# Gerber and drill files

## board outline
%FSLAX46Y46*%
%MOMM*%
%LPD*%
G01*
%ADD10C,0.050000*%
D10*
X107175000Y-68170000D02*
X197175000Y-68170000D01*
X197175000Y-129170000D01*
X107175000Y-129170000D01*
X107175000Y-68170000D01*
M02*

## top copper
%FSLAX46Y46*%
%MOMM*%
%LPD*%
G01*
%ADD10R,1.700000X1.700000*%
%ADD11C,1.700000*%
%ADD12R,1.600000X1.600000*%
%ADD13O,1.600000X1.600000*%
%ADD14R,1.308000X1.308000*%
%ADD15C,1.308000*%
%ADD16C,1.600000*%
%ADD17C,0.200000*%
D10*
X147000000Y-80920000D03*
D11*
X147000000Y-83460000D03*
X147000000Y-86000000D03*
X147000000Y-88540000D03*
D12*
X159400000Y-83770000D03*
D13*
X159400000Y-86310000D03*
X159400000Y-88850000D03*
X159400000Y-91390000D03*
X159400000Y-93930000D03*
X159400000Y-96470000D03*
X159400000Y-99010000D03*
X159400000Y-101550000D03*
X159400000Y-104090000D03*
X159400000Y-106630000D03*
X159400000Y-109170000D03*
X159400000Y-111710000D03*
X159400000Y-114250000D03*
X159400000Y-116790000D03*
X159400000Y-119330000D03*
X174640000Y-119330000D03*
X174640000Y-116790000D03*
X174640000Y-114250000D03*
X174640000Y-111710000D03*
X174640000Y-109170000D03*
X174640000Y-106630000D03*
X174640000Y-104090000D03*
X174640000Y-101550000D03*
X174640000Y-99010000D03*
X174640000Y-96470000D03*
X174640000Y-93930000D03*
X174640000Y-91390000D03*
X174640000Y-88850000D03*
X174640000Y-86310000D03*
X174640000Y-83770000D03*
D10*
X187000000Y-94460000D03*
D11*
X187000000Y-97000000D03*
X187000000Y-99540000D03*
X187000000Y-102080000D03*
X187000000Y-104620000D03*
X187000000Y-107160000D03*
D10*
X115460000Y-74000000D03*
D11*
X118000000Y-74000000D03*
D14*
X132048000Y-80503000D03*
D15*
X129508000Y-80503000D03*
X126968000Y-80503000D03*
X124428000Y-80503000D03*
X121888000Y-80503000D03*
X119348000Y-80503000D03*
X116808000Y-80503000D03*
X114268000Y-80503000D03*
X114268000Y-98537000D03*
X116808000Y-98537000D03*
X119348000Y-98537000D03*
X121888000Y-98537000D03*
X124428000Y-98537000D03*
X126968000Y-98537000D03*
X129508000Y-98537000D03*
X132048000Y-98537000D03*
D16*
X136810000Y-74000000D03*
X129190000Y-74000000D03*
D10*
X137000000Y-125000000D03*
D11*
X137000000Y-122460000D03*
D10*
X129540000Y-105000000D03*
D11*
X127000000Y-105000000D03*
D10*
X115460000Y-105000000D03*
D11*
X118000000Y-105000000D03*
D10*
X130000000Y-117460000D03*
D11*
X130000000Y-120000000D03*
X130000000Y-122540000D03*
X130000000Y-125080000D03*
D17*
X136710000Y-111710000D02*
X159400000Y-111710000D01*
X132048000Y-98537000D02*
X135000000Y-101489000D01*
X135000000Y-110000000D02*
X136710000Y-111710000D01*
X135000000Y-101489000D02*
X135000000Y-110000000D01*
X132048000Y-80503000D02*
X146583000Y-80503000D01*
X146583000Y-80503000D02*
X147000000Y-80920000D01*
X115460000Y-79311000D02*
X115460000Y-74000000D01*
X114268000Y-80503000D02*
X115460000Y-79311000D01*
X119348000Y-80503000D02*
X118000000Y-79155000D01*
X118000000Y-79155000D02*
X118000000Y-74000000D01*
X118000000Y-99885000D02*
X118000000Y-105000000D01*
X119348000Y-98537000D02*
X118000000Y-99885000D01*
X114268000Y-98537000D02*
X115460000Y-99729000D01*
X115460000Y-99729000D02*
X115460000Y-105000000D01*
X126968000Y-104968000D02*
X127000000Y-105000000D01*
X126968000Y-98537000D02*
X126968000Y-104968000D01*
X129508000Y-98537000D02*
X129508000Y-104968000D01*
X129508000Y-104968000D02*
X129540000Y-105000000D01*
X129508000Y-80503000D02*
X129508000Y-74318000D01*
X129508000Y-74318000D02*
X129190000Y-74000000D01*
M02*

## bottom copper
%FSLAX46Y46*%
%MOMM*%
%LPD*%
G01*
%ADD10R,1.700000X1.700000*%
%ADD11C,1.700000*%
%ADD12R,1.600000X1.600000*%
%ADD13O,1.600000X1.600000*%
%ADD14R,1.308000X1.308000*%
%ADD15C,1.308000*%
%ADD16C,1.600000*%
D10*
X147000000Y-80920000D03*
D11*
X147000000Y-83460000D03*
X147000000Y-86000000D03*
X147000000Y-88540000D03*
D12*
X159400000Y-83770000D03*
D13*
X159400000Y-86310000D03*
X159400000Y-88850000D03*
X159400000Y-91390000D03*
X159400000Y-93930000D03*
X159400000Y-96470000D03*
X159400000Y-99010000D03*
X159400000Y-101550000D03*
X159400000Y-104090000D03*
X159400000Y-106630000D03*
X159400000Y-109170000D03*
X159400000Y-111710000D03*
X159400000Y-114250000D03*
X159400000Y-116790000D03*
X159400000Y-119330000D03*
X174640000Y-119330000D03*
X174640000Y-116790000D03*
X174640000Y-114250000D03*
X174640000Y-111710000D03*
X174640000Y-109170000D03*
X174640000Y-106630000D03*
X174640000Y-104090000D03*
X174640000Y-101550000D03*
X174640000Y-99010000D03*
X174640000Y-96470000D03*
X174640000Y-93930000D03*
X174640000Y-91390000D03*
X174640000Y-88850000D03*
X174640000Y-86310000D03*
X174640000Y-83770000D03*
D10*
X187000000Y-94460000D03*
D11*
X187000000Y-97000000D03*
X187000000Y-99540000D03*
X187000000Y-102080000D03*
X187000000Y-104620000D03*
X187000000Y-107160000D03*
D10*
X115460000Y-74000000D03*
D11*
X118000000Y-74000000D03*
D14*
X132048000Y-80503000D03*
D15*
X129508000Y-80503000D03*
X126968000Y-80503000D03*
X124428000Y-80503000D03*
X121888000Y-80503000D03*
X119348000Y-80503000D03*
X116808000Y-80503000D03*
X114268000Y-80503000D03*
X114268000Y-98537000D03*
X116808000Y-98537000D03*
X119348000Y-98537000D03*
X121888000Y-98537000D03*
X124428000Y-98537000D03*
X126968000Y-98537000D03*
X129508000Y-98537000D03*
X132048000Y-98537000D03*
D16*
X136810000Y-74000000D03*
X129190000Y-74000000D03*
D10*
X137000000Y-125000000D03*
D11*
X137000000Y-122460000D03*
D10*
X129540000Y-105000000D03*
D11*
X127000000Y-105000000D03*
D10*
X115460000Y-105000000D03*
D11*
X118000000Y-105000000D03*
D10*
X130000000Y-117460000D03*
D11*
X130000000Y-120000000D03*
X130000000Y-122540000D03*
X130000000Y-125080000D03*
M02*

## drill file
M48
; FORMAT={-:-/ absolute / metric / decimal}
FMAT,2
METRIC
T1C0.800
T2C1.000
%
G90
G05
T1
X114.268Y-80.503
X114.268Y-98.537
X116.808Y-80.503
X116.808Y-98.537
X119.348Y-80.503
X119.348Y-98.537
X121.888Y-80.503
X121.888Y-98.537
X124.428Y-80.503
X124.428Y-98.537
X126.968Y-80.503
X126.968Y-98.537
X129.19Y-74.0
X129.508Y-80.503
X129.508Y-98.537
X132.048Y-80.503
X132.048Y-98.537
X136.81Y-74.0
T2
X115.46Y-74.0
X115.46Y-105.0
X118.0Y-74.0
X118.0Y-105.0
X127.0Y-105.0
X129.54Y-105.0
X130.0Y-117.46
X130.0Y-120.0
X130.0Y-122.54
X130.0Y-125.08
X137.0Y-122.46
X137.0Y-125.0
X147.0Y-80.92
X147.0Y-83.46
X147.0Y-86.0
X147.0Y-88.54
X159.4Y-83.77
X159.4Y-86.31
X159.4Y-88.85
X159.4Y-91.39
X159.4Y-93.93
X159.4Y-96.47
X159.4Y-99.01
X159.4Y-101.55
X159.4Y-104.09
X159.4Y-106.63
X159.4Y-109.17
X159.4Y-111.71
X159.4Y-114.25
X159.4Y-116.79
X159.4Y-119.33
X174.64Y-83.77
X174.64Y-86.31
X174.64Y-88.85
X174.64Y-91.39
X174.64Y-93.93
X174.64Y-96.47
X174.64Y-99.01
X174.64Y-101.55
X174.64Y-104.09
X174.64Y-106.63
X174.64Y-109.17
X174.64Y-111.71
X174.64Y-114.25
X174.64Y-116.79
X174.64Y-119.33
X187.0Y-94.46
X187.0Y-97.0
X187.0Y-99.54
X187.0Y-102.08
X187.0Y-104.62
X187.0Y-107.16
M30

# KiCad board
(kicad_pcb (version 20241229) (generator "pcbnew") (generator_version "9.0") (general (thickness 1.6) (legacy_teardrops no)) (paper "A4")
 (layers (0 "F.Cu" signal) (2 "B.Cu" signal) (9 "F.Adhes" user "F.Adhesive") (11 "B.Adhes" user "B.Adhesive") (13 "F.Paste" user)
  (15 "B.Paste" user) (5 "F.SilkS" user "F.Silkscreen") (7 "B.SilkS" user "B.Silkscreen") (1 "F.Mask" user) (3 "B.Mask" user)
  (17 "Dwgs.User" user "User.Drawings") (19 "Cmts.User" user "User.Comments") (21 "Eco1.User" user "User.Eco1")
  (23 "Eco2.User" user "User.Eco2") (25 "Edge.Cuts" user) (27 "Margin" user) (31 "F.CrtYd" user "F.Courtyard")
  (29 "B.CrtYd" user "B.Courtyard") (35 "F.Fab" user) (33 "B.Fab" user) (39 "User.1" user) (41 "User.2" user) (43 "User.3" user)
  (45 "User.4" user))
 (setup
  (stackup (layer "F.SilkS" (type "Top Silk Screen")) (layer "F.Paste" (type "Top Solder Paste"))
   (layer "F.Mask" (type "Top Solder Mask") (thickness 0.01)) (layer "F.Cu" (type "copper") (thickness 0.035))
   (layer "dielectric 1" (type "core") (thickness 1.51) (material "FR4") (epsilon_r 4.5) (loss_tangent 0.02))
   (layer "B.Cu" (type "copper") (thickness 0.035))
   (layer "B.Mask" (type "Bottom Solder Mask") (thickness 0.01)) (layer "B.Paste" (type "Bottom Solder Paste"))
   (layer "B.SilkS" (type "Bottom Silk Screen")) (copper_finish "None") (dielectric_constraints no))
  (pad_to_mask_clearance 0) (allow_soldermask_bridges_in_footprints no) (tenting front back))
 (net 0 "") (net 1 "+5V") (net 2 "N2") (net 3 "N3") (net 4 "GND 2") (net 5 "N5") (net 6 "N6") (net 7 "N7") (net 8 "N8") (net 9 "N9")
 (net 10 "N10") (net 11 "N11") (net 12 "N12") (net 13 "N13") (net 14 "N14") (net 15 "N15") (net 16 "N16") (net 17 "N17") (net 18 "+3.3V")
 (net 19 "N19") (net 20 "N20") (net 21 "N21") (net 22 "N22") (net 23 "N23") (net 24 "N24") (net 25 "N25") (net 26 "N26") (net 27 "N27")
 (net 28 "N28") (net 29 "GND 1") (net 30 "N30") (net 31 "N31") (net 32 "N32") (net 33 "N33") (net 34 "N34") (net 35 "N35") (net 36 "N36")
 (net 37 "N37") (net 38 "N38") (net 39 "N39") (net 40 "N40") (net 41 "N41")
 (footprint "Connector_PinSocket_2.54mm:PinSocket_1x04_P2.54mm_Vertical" (layer "F.Cu") (at 147 80.92)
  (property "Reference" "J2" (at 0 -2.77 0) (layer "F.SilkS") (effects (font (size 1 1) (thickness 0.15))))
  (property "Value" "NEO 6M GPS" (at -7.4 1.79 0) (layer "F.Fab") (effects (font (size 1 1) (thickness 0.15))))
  (pad "1" thru_hole rect (at 0 0) (size 1.7 1.7) (drill 1) (layers "*.Cu" "*.Mask") (remove_unused_layers no) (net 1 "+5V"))
  (pad "2" thru_hole circle (at 0 2.54) (size 1.7 1.7) (drill 1) (layers "*.Cu" "*.Mask") (remove_unused_layers no) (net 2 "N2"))
  (pad "3" thru_hole circle (at 0 5.08) (size 1.7 1.7) (drill 1) (layers "*.Cu" "*.Mask") (remove_unused_layers no) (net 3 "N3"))
  (pad "4" thru_hole circle (at 0 7.62) (size 1.7 1.7) (drill 1) (layers "*.Cu" "*.Mask") (remove_unused_layers no) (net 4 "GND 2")))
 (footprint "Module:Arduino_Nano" (layer "F.Cu") (at 159.4 83.77)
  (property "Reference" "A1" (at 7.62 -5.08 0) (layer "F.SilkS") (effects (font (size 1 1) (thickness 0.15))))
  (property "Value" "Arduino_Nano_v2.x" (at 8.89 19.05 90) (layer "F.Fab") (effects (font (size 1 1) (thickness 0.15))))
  (pad "1" thru_hole rect (at 0 0) (size 1.6 1.6) (drill 1) (layers "*.Cu" "*.Mask") (remove_unused_layers no) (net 2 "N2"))
  (pad "2" thru_hole oval (at 0 2.54) (size 1.6 1.6) (drill 1) (layers "*.Cu" "*.Mask") (remove_unused_layers no) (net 3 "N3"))
  (pad "3" thru_hole oval (at 0 5.08) (size 1.6 1.6) (drill 1) (layers "*.Cu" "*.Mask") (remove_unused_layers no) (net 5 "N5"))
  (pad "4" thru_hole oval (at 0 7.62) (size 1.6 1.6) (drill 1) (layers "*.Cu" "*.Mask") (remove_unused_layers no) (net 4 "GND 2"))
  (pad "5" thru_hole oval (at 0 10.16) (size 1.6 1.6) (drill 1) (layers "*.Cu" "*.Mask") (remove_unused_layers no) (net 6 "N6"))
  (pad "6" thru_hole oval (at 0 12.7) (size 1.6 1.6) (drill 1) (layers "*.Cu" "*.Mask") (remove_unused_layers no) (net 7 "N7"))
  (pad "7" thru_hole oval (at 0 15.24) (size 1.6 1.6) (drill 1) (layers "*.Cu" "*.Mask") (remove_unused_layers no) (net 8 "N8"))
  (pad "8" thru_hole oval (at 0 17.78) (size 1.6 1.6) (drill 1) (layers "*.Cu" "*.Mask") (remove_unused_layers no) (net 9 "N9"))
  (pad "9" thru_hole oval (at 0 20.32) (size 1.6 1.6) (drill 1) (layers "*.Cu" "*.Mask") (remove_unused_layers no) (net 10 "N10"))
  (pad "10" thru_hole oval (at 0 22.86) (size 1.6 1.6) (drill 1) (layers "*.Cu" "*.Mask") (remove_unused_layers no) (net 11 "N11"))
  (pad "11" thru_hole oval (at 0 25.4) (size 1.6 1.6) (drill 1) (layers "*.Cu" "*.Mask") (remove_unused_layers no) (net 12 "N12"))
  (pad "12" thru_hole oval (at 0 27.94) (size 1.6 1.6) (drill 1) (layers "*.Cu" "*.Mask") (remove_unused_layers no) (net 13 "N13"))
  (pad "13" thru_hole oval (at 0 30.48) (size 1.6 1.6) (drill 1) (layers "*.Cu" "*.Mask") (remove_unused_layers no) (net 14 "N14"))
  (pad "14" thru_hole oval (at 0 33.02) (size 1.6 1.6) (drill 1) (layers "*.Cu" "*.Mask") (remove_unused_layers no) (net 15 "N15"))
  (pad "15" thru_hole oval (at 0 35.56) (size 1.6 1.6) (drill 1) (layers "*.Cu" "*.Mask") (remove_unused_layers no) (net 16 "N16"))
  (pad "16" thru_hole oval (at 15.24 35.56) (size 1.6 1.6) (drill 1) (layers "*.Cu" "*.Mask") (remove_unused_layers no) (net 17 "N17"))
  (pad "17" thru_hole oval (at 15.24 33.02) (size 1.6 1.6) (drill 1) (layers "*.Cu" "*.Mask") (remove_unused_layers no) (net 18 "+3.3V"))
  (pad "18" thru_hole oval (at 15.24 30.48) (size 1.6 1.6) (drill 1) (layers "*.Cu" "*.Mask") (remove_unused_layers no) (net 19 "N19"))
  (pad "19" thru_hole oval (at 15.24 27.94) (size 1.6 1.6) (drill 1) (layers "*.Cu" "*.Mask") (remove_unused_layers no) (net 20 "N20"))
  (pad "20" thru_hole oval (at 15.24 25.4) (size 1.6 1.6) (drill 1) (layers "*.Cu" "*.Mask") (remove_unused_layers no) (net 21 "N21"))
  (pad "21" thru_hole oval (at 15.24 22.86) (size 1.6 1.6) (drill 1) (layers "*.Cu" "*.Mask") (remove_unused_layers no) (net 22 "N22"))
  (pad "22" thru_hole oval (at 15.24 20.32) (size 1.6 1.6) (drill 1) (layers "*.Cu" "*.Mask") (remove_unused_layers no) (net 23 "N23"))
  (pad "23" thru_hole oval (at 15.24 17.78) (size 1.6 1.6) (drill 1) (layers "*.Cu" "*.Mask") (remove_unused_layers no) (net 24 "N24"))
  (pad "24" thru_hole oval (at 15.24 15.24) (size 1.6 1.6) (drill 1) (layers "*.Cu" "*.Mask") (remove_unused_layers no) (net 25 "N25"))
  (pad "25" thru_hole oval (at 15.24 12.7) (size 1.6 1.6) (drill 1) (layers "*.Cu" "*.Mask") (remove_unused_layers no) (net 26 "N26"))
  (pad "26" thru_hole oval (at 15.24 10.16) (size 1.6 1.6) (drill 1) (layers "*.Cu" "*.Mask") (remove_unused_layers no) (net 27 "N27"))
  (pad "27" thru_hole oval (at 15.24 7.62) (size 1.6 1.6) (drill 1) (layers "*.Cu" "*.Mask") (remove_unused_layers no) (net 1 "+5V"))
  (pad "28" thru_hole oval (at 15.24 5.08) (size 1.6 1.6) (drill 1) (layers "*.Cu" "*.Mask") (remove_unused_layers no) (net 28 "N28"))
  (pad "29" thru_hole oval (at 15.24 2.54) (size 1.6 1.6) (drill 1) (layers "*.Cu" "*.Mask") (remove_unused_layers no) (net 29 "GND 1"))
  (pad "30" thru_hole oval (at 15.24 0) (size 1.6 1.6) (drill 1) (layers "*.Cu" "*.Mask") (remove_unused_layers no) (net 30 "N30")))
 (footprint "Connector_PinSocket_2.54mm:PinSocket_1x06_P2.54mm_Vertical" (layer "F.Cu") (at 187 94.46)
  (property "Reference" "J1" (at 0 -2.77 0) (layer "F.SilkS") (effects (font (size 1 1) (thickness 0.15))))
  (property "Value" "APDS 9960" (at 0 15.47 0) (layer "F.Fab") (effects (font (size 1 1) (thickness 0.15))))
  (pad "1" thru_hole rect (at 0 0) (size 1.7 1.7) (drill 1) (layers "*.Cu" "*.Mask") (remove_unused_layers no) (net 18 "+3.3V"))
  (pad "2" thru_hole circle (at 0 2.54) (size 1.7 1.7) (drill 1) (layers "*.Cu" "*.Mask") (remove_unused_layers no) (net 29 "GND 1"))
  (pad "3" thru_hole circle (at 0 5.08) (size 1.7 1.7) (drill 1) (layers "*.Cu" "*.Mask") (remove_unused_layers no) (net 1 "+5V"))
  (pad "4" thru_hole circle (at 0 7.62) (size 1.7 1.7) (drill 1) (layers "*.Cu" "*.Mask") (remove_unused_layers no) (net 24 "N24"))
  (pad "5" thru_hole circle (at 0 10.16) (size 1.7 1.7) (drill 1) (layers "*.Cu" "*.Mask") (remove_unused_layers no) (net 25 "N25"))
  (pad "6" thru_hole circle (at 0 12.7) (size 1.7 1.7) (drill 1) (layers "*.Cu" "*.Mask") (remove_unused_layers no) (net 6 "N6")))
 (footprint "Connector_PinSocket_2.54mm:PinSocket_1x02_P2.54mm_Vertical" (layer "F.Cu") (at 115.46 74 90)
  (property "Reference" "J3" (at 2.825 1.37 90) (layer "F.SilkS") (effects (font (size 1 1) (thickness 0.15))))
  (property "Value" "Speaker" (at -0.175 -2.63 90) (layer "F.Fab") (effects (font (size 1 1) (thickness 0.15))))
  (pad "1" thru_hole rect (at 0 0 90) (size 1.7 1.7) (drill 1) (layers "*.Cu" "*.Mask") (remove_unused_layers no) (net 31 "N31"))
  (pad "2" thru_hole circle (at 0 2.54 90) (size 1.7 1.7) (drill 1) (layers "*.Cu" "*.Mask") (remove_unused_layers no) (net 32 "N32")))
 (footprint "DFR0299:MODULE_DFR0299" (layer "F.Cu") (at 123.158 89.52 -90)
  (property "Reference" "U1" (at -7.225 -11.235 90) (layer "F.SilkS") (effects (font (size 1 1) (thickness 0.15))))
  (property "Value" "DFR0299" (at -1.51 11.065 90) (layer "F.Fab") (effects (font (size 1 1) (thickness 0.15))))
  (pad "1" thru_hole rect (at -9.017 -8.89 270) (size 1.308 1.308) (drill 0.8) (layers "*.Cu" "*.Mask") (remove_unused_layers no)
   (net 1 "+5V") (solder_mask_margin 0.102))
  (pad "2" thru_hole circle (at -9.017 -6.35 270) (size 1.308 1.308) (drill 0.8) (layers "*.Cu" "*.Mask") (remove_unused_layers no)
   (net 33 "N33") (solder_mask_margin 0.102))
  (pad "3" thru_hole circle (at -9.017 -3.81 270) (size 1.308 1.308) (drill 0.8) (layers "*.Cu" "*.Mask") (remove_unused_layers no)
   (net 14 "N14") (solder_mask_margin 0.102))
  (pad "4" thru_hole circle (at -9.017 -1.27 270) (size 1.308 1.308) (drill 0.8) (layers "*.Cu" "*.Mask") (remove_unused_layers no)
   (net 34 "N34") (solder_mask_margin 0.102))
  (pad "5" thru_hole circle (at -9.017 1.27 270) (size 1.308 1.308) (drill 0.8) (layers "*.Cu" "*.Mask") (remove_unused_layers no)
   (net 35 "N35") (solder_mask_margin 0.102))
  (pad "6" thru_hole circle (at -9.017 3.81 270) (size 1.308 1.308) (drill 0.8) (layers "*.Cu" "*.Mask") (remove_unused_layers no)
   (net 32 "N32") (solder_mask_margin 0.102))
  (pad "7" thru_hole circle (at -9.017 6.35 270) (size 1.308 1.308) (drill 0.8) (layers "*.Cu" "*.Mask") (remove_unused_layers no)
   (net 4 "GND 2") (solder_mask_margin 0.102))
  (pad "8" thru_hole circle (at -9.017 8.89 270) (size 1.308 1.308) (drill 0.8) (layers "*.Cu" "*.Mask") (remove_unused_layers no)
   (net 31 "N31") (solder_mask_margin 0.102))
  (pad "9" thru_hole circle (at 9.017 8.89 270) (size 1.308 1.308) (drill 0.8) (layers "*.Cu" "*.Mask") (remove_unused_layers no)
   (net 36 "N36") (solder_mask_margin 0.102))
  (pad "10" thru_hole circle (at 9.017 6.35 270) (size 1.308 1.308) (drill 0.8) (layers "*.Cu" "*.Mask") (remove_unused_layers no)
   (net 4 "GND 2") (solder_mask_margin 0.102))
  (pad "11" thru_hole circle (at 9.017 3.81 270) (size 1.308 1.308) (drill 0.8) (layers "*.Cu" "*.Mask") (remove_unused_layers no)
   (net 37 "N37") (solder_mask_margin 0.102))
  (pad "12" thru_hole circle (at 9.017 1.27 270) (size 1.308 1.308) (drill 0.8) (layers "*.Cu" "*.Mask") (remove_unused_layers no)
   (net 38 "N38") (solder_mask_margin 0.102))
  (pad "13" thru_hole circle (at 9.017 -1.27 270) (size 1.308 1.308) (drill 0.8) (layers "*.Cu" "*.Mask") (remove_unused_layers no)
   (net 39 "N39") (solder_mask_margin 0.102))
  (pad "14" thru_hole circle (at 9.017 -3.81 270) (size 1.308 1.308) (drill 0.8) (layers "*.Cu" "*.Mask") (remove_unused_layers no)
   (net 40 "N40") (solder_mask_margin 0.102))
  (pad "15" thru_hole circle (at 9.017 -6.35 270) (size 1.308 1.308) (drill 0.8) (layers "*.Cu" "*.Mask") (remove_unused_layers no)
   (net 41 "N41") (solder_mask_margin 0.102))
  (pad "16" thru_hole circle (at 9.017 -8.89 270) (size 1.308 1.308) (drill 0.8) (layers "*.Cu" "*.Mask") (remove_unused_layers no)
   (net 13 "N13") (solder_mask_margin 0.102)))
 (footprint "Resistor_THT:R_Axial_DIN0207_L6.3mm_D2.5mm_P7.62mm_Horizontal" (layer "F.Cu") (at 136.81 74 180)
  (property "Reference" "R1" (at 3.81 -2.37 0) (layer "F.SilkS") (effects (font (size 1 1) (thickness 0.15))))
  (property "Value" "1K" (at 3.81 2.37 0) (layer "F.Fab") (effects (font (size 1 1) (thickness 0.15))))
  (pad "1" thru_hole circle (at 0 0 180) (size 1.6 1.6) (drill 0.8) (layers "*.Cu" "*.Mask") (remove_unused_layers no) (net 15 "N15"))
  (pad "2" thru_hole circle (at 7.62 0 180) (size 1.6 1.6) (drill 0.8) (layers "*.Cu" "*.Mask") (remove_unused_layers no) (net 33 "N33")))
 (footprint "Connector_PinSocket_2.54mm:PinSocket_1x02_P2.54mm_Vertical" (layer "B.Cu") (at 137 125)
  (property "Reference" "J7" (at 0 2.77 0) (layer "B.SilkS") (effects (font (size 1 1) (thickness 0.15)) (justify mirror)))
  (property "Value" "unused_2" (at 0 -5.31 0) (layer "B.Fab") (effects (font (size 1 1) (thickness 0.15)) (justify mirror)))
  (pad "1" thru_hole rect (at 0 0) (size 1.7 1.7) (drill 1) (layers "*.Cu" "*.Mask") (remove_unused_layers no) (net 12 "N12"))
  (pad "2" thru_hole circle (at 0 -2.54) (size 1.7 1.7) (drill 1) (layers "*.Cu" "*.Mask") (remove_unused_layers no) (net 11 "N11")))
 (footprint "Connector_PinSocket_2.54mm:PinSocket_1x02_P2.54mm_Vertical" (layer "B.Cu") (at 129.54 105 90)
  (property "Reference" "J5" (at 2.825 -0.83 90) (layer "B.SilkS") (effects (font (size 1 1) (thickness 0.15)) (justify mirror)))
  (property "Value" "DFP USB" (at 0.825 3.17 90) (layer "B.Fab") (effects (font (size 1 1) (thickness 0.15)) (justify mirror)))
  (pad "1" thru_hole rect (at 0 0 90) (size 1.7 1.7) (drill 1) (layers "*.Cu" "*.Mask") (remove_unused_layers no) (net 41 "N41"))
  (pad "2" thru_hole circle (at 0 -2.54 90) (size 1.7 1.7) (drill 1) (layers "*.Cu" "*.Mask") (remove_unused_layers no) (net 40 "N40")))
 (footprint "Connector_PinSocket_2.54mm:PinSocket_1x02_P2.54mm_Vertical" (layer "B.Cu") (at 115.46 105 -90)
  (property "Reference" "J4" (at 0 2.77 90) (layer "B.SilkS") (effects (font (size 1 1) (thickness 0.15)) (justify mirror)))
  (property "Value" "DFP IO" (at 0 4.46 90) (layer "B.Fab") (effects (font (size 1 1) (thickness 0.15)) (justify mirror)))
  (pad "1" thru_hole rect (at 0 0 270) (size 1.7 1.7) (drill 1) (layers "*.Cu" "*.Mask") (remove_unused_layers no) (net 36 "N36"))
  (pad "2" thru_hole circle (at 0 -2.54 270) (size 1.7 1.7) (drill 1) (layers "*.Cu" "*.Mask") (remove_unused_layers no) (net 37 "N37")))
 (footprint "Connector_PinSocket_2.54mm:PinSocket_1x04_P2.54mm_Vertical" (layer "B.Cu") (at 130 117.46 180)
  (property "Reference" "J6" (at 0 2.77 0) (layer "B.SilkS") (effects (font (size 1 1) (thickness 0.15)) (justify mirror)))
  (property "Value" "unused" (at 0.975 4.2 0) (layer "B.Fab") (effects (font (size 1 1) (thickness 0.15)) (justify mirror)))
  (pad "1" thru_hole rect (at 0 0 180) (size 1.7 1.7) (drill 1) (layers "*.Cu" "*.Mask") (remove_unused_layers no) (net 10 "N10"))
  (pad "2" thru_hole circle (at 0 -2.54 180) (size 1.7 1.7) (drill 1) (layers "*.Cu" "*.Mask") (remove_unused_layers no) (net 9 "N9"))
  (pad "3" thru_hole circle (at 0 -5.08 180) (size 1.7 1.7) (drill 1) (layers "*.Cu" "*.Mask") (remove_unused_layers no) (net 8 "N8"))
  (pad "4" thru_hole circle (at 0 -7.62 180) (size 1.7 1.7) (drill 1) (layers "*.Cu" "*.Mask") (remove_unused_layers no) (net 7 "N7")))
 (gr_rect (start 107.175 68.17) (end 197.175 129.17) (stroke (width 0.05) (type default)) (fill no) (layer "Edge.Cuts"))
 (segment (start 136.71 111.71) (end 159.4 111.71) (width 0.2) (layer "F.Cu") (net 13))
 (segment (start 132.048 98.537) (end 135 101.489) (width 0.2) (layer "F.Cu") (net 13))
 (segment (start 135 110) (end 136.71 111.71) (width 0.2) (layer "F.Cu") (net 13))
 (segment (start 135 101.489) (end 135 110) (width 0.2) (layer "F.Cu") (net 13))
 (segment (start 132.048 80.503) (end 146.583 80.503) (width 0.2) (layer "F.Cu") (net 1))
 (segment (start 146.583 80.503) (end 147 80.92) (width 0.2) (layer "F.Cu") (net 1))
 (segment (start 115.46 79.311) (end 115.46 74) (width 0.2) (layer "F.Cu") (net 31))
 (segment (start 114.268 80.503) (end 115.46 79.311) (width 0.2) (layer "F.Cu") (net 31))
 (segment (start 119.348 80.503) (end 118 79.155) (width 0.2) (layer "F.Cu") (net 32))
 (segment (start 118 79.155) (end 118 74) (width 0.2) (layer "F.Cu") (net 32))
 (segment (start 118 99.885) (end 118 105) (width 0.2) (layer "F.Cu") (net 37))
 (segment (start 119.348 98.537) (end 118 99.885) (width 0.2) (layer "F.Cu") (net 37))
 (segment (start 114.268 98.537) (end 115.46 99.729) (width 0.2) (layer "F.Cu") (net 36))
 (segment (start 115.46 99.729) (end 115.46 105) (width 0.2) (layer "F.Cu") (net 36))
 (segment (start 126.968 104.968) (end 127 105) (width 0.2) (layer "F.Cu") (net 40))
 (segment (start 126.968 98.537) (end 126.968 104.968) (width 0.2) (layer "F.Cu") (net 40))
 (segment (start 129.508 98.537) (end 129.508 104.968) (width 0.2) (layer "F.Cu") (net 41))
 (segment (start 129.508 104.968) (end 129.54 105) (width 0.2) (layer "F.Cu") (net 41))
 (segment (start 129.508 80.503) (end 129.508 74.318) (width 0.2) (layer "F.Cu") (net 33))
 (segment (start 129.508 74.318) (end 129.19 74) (width 0.2) (layer "F.Cu") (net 33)))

